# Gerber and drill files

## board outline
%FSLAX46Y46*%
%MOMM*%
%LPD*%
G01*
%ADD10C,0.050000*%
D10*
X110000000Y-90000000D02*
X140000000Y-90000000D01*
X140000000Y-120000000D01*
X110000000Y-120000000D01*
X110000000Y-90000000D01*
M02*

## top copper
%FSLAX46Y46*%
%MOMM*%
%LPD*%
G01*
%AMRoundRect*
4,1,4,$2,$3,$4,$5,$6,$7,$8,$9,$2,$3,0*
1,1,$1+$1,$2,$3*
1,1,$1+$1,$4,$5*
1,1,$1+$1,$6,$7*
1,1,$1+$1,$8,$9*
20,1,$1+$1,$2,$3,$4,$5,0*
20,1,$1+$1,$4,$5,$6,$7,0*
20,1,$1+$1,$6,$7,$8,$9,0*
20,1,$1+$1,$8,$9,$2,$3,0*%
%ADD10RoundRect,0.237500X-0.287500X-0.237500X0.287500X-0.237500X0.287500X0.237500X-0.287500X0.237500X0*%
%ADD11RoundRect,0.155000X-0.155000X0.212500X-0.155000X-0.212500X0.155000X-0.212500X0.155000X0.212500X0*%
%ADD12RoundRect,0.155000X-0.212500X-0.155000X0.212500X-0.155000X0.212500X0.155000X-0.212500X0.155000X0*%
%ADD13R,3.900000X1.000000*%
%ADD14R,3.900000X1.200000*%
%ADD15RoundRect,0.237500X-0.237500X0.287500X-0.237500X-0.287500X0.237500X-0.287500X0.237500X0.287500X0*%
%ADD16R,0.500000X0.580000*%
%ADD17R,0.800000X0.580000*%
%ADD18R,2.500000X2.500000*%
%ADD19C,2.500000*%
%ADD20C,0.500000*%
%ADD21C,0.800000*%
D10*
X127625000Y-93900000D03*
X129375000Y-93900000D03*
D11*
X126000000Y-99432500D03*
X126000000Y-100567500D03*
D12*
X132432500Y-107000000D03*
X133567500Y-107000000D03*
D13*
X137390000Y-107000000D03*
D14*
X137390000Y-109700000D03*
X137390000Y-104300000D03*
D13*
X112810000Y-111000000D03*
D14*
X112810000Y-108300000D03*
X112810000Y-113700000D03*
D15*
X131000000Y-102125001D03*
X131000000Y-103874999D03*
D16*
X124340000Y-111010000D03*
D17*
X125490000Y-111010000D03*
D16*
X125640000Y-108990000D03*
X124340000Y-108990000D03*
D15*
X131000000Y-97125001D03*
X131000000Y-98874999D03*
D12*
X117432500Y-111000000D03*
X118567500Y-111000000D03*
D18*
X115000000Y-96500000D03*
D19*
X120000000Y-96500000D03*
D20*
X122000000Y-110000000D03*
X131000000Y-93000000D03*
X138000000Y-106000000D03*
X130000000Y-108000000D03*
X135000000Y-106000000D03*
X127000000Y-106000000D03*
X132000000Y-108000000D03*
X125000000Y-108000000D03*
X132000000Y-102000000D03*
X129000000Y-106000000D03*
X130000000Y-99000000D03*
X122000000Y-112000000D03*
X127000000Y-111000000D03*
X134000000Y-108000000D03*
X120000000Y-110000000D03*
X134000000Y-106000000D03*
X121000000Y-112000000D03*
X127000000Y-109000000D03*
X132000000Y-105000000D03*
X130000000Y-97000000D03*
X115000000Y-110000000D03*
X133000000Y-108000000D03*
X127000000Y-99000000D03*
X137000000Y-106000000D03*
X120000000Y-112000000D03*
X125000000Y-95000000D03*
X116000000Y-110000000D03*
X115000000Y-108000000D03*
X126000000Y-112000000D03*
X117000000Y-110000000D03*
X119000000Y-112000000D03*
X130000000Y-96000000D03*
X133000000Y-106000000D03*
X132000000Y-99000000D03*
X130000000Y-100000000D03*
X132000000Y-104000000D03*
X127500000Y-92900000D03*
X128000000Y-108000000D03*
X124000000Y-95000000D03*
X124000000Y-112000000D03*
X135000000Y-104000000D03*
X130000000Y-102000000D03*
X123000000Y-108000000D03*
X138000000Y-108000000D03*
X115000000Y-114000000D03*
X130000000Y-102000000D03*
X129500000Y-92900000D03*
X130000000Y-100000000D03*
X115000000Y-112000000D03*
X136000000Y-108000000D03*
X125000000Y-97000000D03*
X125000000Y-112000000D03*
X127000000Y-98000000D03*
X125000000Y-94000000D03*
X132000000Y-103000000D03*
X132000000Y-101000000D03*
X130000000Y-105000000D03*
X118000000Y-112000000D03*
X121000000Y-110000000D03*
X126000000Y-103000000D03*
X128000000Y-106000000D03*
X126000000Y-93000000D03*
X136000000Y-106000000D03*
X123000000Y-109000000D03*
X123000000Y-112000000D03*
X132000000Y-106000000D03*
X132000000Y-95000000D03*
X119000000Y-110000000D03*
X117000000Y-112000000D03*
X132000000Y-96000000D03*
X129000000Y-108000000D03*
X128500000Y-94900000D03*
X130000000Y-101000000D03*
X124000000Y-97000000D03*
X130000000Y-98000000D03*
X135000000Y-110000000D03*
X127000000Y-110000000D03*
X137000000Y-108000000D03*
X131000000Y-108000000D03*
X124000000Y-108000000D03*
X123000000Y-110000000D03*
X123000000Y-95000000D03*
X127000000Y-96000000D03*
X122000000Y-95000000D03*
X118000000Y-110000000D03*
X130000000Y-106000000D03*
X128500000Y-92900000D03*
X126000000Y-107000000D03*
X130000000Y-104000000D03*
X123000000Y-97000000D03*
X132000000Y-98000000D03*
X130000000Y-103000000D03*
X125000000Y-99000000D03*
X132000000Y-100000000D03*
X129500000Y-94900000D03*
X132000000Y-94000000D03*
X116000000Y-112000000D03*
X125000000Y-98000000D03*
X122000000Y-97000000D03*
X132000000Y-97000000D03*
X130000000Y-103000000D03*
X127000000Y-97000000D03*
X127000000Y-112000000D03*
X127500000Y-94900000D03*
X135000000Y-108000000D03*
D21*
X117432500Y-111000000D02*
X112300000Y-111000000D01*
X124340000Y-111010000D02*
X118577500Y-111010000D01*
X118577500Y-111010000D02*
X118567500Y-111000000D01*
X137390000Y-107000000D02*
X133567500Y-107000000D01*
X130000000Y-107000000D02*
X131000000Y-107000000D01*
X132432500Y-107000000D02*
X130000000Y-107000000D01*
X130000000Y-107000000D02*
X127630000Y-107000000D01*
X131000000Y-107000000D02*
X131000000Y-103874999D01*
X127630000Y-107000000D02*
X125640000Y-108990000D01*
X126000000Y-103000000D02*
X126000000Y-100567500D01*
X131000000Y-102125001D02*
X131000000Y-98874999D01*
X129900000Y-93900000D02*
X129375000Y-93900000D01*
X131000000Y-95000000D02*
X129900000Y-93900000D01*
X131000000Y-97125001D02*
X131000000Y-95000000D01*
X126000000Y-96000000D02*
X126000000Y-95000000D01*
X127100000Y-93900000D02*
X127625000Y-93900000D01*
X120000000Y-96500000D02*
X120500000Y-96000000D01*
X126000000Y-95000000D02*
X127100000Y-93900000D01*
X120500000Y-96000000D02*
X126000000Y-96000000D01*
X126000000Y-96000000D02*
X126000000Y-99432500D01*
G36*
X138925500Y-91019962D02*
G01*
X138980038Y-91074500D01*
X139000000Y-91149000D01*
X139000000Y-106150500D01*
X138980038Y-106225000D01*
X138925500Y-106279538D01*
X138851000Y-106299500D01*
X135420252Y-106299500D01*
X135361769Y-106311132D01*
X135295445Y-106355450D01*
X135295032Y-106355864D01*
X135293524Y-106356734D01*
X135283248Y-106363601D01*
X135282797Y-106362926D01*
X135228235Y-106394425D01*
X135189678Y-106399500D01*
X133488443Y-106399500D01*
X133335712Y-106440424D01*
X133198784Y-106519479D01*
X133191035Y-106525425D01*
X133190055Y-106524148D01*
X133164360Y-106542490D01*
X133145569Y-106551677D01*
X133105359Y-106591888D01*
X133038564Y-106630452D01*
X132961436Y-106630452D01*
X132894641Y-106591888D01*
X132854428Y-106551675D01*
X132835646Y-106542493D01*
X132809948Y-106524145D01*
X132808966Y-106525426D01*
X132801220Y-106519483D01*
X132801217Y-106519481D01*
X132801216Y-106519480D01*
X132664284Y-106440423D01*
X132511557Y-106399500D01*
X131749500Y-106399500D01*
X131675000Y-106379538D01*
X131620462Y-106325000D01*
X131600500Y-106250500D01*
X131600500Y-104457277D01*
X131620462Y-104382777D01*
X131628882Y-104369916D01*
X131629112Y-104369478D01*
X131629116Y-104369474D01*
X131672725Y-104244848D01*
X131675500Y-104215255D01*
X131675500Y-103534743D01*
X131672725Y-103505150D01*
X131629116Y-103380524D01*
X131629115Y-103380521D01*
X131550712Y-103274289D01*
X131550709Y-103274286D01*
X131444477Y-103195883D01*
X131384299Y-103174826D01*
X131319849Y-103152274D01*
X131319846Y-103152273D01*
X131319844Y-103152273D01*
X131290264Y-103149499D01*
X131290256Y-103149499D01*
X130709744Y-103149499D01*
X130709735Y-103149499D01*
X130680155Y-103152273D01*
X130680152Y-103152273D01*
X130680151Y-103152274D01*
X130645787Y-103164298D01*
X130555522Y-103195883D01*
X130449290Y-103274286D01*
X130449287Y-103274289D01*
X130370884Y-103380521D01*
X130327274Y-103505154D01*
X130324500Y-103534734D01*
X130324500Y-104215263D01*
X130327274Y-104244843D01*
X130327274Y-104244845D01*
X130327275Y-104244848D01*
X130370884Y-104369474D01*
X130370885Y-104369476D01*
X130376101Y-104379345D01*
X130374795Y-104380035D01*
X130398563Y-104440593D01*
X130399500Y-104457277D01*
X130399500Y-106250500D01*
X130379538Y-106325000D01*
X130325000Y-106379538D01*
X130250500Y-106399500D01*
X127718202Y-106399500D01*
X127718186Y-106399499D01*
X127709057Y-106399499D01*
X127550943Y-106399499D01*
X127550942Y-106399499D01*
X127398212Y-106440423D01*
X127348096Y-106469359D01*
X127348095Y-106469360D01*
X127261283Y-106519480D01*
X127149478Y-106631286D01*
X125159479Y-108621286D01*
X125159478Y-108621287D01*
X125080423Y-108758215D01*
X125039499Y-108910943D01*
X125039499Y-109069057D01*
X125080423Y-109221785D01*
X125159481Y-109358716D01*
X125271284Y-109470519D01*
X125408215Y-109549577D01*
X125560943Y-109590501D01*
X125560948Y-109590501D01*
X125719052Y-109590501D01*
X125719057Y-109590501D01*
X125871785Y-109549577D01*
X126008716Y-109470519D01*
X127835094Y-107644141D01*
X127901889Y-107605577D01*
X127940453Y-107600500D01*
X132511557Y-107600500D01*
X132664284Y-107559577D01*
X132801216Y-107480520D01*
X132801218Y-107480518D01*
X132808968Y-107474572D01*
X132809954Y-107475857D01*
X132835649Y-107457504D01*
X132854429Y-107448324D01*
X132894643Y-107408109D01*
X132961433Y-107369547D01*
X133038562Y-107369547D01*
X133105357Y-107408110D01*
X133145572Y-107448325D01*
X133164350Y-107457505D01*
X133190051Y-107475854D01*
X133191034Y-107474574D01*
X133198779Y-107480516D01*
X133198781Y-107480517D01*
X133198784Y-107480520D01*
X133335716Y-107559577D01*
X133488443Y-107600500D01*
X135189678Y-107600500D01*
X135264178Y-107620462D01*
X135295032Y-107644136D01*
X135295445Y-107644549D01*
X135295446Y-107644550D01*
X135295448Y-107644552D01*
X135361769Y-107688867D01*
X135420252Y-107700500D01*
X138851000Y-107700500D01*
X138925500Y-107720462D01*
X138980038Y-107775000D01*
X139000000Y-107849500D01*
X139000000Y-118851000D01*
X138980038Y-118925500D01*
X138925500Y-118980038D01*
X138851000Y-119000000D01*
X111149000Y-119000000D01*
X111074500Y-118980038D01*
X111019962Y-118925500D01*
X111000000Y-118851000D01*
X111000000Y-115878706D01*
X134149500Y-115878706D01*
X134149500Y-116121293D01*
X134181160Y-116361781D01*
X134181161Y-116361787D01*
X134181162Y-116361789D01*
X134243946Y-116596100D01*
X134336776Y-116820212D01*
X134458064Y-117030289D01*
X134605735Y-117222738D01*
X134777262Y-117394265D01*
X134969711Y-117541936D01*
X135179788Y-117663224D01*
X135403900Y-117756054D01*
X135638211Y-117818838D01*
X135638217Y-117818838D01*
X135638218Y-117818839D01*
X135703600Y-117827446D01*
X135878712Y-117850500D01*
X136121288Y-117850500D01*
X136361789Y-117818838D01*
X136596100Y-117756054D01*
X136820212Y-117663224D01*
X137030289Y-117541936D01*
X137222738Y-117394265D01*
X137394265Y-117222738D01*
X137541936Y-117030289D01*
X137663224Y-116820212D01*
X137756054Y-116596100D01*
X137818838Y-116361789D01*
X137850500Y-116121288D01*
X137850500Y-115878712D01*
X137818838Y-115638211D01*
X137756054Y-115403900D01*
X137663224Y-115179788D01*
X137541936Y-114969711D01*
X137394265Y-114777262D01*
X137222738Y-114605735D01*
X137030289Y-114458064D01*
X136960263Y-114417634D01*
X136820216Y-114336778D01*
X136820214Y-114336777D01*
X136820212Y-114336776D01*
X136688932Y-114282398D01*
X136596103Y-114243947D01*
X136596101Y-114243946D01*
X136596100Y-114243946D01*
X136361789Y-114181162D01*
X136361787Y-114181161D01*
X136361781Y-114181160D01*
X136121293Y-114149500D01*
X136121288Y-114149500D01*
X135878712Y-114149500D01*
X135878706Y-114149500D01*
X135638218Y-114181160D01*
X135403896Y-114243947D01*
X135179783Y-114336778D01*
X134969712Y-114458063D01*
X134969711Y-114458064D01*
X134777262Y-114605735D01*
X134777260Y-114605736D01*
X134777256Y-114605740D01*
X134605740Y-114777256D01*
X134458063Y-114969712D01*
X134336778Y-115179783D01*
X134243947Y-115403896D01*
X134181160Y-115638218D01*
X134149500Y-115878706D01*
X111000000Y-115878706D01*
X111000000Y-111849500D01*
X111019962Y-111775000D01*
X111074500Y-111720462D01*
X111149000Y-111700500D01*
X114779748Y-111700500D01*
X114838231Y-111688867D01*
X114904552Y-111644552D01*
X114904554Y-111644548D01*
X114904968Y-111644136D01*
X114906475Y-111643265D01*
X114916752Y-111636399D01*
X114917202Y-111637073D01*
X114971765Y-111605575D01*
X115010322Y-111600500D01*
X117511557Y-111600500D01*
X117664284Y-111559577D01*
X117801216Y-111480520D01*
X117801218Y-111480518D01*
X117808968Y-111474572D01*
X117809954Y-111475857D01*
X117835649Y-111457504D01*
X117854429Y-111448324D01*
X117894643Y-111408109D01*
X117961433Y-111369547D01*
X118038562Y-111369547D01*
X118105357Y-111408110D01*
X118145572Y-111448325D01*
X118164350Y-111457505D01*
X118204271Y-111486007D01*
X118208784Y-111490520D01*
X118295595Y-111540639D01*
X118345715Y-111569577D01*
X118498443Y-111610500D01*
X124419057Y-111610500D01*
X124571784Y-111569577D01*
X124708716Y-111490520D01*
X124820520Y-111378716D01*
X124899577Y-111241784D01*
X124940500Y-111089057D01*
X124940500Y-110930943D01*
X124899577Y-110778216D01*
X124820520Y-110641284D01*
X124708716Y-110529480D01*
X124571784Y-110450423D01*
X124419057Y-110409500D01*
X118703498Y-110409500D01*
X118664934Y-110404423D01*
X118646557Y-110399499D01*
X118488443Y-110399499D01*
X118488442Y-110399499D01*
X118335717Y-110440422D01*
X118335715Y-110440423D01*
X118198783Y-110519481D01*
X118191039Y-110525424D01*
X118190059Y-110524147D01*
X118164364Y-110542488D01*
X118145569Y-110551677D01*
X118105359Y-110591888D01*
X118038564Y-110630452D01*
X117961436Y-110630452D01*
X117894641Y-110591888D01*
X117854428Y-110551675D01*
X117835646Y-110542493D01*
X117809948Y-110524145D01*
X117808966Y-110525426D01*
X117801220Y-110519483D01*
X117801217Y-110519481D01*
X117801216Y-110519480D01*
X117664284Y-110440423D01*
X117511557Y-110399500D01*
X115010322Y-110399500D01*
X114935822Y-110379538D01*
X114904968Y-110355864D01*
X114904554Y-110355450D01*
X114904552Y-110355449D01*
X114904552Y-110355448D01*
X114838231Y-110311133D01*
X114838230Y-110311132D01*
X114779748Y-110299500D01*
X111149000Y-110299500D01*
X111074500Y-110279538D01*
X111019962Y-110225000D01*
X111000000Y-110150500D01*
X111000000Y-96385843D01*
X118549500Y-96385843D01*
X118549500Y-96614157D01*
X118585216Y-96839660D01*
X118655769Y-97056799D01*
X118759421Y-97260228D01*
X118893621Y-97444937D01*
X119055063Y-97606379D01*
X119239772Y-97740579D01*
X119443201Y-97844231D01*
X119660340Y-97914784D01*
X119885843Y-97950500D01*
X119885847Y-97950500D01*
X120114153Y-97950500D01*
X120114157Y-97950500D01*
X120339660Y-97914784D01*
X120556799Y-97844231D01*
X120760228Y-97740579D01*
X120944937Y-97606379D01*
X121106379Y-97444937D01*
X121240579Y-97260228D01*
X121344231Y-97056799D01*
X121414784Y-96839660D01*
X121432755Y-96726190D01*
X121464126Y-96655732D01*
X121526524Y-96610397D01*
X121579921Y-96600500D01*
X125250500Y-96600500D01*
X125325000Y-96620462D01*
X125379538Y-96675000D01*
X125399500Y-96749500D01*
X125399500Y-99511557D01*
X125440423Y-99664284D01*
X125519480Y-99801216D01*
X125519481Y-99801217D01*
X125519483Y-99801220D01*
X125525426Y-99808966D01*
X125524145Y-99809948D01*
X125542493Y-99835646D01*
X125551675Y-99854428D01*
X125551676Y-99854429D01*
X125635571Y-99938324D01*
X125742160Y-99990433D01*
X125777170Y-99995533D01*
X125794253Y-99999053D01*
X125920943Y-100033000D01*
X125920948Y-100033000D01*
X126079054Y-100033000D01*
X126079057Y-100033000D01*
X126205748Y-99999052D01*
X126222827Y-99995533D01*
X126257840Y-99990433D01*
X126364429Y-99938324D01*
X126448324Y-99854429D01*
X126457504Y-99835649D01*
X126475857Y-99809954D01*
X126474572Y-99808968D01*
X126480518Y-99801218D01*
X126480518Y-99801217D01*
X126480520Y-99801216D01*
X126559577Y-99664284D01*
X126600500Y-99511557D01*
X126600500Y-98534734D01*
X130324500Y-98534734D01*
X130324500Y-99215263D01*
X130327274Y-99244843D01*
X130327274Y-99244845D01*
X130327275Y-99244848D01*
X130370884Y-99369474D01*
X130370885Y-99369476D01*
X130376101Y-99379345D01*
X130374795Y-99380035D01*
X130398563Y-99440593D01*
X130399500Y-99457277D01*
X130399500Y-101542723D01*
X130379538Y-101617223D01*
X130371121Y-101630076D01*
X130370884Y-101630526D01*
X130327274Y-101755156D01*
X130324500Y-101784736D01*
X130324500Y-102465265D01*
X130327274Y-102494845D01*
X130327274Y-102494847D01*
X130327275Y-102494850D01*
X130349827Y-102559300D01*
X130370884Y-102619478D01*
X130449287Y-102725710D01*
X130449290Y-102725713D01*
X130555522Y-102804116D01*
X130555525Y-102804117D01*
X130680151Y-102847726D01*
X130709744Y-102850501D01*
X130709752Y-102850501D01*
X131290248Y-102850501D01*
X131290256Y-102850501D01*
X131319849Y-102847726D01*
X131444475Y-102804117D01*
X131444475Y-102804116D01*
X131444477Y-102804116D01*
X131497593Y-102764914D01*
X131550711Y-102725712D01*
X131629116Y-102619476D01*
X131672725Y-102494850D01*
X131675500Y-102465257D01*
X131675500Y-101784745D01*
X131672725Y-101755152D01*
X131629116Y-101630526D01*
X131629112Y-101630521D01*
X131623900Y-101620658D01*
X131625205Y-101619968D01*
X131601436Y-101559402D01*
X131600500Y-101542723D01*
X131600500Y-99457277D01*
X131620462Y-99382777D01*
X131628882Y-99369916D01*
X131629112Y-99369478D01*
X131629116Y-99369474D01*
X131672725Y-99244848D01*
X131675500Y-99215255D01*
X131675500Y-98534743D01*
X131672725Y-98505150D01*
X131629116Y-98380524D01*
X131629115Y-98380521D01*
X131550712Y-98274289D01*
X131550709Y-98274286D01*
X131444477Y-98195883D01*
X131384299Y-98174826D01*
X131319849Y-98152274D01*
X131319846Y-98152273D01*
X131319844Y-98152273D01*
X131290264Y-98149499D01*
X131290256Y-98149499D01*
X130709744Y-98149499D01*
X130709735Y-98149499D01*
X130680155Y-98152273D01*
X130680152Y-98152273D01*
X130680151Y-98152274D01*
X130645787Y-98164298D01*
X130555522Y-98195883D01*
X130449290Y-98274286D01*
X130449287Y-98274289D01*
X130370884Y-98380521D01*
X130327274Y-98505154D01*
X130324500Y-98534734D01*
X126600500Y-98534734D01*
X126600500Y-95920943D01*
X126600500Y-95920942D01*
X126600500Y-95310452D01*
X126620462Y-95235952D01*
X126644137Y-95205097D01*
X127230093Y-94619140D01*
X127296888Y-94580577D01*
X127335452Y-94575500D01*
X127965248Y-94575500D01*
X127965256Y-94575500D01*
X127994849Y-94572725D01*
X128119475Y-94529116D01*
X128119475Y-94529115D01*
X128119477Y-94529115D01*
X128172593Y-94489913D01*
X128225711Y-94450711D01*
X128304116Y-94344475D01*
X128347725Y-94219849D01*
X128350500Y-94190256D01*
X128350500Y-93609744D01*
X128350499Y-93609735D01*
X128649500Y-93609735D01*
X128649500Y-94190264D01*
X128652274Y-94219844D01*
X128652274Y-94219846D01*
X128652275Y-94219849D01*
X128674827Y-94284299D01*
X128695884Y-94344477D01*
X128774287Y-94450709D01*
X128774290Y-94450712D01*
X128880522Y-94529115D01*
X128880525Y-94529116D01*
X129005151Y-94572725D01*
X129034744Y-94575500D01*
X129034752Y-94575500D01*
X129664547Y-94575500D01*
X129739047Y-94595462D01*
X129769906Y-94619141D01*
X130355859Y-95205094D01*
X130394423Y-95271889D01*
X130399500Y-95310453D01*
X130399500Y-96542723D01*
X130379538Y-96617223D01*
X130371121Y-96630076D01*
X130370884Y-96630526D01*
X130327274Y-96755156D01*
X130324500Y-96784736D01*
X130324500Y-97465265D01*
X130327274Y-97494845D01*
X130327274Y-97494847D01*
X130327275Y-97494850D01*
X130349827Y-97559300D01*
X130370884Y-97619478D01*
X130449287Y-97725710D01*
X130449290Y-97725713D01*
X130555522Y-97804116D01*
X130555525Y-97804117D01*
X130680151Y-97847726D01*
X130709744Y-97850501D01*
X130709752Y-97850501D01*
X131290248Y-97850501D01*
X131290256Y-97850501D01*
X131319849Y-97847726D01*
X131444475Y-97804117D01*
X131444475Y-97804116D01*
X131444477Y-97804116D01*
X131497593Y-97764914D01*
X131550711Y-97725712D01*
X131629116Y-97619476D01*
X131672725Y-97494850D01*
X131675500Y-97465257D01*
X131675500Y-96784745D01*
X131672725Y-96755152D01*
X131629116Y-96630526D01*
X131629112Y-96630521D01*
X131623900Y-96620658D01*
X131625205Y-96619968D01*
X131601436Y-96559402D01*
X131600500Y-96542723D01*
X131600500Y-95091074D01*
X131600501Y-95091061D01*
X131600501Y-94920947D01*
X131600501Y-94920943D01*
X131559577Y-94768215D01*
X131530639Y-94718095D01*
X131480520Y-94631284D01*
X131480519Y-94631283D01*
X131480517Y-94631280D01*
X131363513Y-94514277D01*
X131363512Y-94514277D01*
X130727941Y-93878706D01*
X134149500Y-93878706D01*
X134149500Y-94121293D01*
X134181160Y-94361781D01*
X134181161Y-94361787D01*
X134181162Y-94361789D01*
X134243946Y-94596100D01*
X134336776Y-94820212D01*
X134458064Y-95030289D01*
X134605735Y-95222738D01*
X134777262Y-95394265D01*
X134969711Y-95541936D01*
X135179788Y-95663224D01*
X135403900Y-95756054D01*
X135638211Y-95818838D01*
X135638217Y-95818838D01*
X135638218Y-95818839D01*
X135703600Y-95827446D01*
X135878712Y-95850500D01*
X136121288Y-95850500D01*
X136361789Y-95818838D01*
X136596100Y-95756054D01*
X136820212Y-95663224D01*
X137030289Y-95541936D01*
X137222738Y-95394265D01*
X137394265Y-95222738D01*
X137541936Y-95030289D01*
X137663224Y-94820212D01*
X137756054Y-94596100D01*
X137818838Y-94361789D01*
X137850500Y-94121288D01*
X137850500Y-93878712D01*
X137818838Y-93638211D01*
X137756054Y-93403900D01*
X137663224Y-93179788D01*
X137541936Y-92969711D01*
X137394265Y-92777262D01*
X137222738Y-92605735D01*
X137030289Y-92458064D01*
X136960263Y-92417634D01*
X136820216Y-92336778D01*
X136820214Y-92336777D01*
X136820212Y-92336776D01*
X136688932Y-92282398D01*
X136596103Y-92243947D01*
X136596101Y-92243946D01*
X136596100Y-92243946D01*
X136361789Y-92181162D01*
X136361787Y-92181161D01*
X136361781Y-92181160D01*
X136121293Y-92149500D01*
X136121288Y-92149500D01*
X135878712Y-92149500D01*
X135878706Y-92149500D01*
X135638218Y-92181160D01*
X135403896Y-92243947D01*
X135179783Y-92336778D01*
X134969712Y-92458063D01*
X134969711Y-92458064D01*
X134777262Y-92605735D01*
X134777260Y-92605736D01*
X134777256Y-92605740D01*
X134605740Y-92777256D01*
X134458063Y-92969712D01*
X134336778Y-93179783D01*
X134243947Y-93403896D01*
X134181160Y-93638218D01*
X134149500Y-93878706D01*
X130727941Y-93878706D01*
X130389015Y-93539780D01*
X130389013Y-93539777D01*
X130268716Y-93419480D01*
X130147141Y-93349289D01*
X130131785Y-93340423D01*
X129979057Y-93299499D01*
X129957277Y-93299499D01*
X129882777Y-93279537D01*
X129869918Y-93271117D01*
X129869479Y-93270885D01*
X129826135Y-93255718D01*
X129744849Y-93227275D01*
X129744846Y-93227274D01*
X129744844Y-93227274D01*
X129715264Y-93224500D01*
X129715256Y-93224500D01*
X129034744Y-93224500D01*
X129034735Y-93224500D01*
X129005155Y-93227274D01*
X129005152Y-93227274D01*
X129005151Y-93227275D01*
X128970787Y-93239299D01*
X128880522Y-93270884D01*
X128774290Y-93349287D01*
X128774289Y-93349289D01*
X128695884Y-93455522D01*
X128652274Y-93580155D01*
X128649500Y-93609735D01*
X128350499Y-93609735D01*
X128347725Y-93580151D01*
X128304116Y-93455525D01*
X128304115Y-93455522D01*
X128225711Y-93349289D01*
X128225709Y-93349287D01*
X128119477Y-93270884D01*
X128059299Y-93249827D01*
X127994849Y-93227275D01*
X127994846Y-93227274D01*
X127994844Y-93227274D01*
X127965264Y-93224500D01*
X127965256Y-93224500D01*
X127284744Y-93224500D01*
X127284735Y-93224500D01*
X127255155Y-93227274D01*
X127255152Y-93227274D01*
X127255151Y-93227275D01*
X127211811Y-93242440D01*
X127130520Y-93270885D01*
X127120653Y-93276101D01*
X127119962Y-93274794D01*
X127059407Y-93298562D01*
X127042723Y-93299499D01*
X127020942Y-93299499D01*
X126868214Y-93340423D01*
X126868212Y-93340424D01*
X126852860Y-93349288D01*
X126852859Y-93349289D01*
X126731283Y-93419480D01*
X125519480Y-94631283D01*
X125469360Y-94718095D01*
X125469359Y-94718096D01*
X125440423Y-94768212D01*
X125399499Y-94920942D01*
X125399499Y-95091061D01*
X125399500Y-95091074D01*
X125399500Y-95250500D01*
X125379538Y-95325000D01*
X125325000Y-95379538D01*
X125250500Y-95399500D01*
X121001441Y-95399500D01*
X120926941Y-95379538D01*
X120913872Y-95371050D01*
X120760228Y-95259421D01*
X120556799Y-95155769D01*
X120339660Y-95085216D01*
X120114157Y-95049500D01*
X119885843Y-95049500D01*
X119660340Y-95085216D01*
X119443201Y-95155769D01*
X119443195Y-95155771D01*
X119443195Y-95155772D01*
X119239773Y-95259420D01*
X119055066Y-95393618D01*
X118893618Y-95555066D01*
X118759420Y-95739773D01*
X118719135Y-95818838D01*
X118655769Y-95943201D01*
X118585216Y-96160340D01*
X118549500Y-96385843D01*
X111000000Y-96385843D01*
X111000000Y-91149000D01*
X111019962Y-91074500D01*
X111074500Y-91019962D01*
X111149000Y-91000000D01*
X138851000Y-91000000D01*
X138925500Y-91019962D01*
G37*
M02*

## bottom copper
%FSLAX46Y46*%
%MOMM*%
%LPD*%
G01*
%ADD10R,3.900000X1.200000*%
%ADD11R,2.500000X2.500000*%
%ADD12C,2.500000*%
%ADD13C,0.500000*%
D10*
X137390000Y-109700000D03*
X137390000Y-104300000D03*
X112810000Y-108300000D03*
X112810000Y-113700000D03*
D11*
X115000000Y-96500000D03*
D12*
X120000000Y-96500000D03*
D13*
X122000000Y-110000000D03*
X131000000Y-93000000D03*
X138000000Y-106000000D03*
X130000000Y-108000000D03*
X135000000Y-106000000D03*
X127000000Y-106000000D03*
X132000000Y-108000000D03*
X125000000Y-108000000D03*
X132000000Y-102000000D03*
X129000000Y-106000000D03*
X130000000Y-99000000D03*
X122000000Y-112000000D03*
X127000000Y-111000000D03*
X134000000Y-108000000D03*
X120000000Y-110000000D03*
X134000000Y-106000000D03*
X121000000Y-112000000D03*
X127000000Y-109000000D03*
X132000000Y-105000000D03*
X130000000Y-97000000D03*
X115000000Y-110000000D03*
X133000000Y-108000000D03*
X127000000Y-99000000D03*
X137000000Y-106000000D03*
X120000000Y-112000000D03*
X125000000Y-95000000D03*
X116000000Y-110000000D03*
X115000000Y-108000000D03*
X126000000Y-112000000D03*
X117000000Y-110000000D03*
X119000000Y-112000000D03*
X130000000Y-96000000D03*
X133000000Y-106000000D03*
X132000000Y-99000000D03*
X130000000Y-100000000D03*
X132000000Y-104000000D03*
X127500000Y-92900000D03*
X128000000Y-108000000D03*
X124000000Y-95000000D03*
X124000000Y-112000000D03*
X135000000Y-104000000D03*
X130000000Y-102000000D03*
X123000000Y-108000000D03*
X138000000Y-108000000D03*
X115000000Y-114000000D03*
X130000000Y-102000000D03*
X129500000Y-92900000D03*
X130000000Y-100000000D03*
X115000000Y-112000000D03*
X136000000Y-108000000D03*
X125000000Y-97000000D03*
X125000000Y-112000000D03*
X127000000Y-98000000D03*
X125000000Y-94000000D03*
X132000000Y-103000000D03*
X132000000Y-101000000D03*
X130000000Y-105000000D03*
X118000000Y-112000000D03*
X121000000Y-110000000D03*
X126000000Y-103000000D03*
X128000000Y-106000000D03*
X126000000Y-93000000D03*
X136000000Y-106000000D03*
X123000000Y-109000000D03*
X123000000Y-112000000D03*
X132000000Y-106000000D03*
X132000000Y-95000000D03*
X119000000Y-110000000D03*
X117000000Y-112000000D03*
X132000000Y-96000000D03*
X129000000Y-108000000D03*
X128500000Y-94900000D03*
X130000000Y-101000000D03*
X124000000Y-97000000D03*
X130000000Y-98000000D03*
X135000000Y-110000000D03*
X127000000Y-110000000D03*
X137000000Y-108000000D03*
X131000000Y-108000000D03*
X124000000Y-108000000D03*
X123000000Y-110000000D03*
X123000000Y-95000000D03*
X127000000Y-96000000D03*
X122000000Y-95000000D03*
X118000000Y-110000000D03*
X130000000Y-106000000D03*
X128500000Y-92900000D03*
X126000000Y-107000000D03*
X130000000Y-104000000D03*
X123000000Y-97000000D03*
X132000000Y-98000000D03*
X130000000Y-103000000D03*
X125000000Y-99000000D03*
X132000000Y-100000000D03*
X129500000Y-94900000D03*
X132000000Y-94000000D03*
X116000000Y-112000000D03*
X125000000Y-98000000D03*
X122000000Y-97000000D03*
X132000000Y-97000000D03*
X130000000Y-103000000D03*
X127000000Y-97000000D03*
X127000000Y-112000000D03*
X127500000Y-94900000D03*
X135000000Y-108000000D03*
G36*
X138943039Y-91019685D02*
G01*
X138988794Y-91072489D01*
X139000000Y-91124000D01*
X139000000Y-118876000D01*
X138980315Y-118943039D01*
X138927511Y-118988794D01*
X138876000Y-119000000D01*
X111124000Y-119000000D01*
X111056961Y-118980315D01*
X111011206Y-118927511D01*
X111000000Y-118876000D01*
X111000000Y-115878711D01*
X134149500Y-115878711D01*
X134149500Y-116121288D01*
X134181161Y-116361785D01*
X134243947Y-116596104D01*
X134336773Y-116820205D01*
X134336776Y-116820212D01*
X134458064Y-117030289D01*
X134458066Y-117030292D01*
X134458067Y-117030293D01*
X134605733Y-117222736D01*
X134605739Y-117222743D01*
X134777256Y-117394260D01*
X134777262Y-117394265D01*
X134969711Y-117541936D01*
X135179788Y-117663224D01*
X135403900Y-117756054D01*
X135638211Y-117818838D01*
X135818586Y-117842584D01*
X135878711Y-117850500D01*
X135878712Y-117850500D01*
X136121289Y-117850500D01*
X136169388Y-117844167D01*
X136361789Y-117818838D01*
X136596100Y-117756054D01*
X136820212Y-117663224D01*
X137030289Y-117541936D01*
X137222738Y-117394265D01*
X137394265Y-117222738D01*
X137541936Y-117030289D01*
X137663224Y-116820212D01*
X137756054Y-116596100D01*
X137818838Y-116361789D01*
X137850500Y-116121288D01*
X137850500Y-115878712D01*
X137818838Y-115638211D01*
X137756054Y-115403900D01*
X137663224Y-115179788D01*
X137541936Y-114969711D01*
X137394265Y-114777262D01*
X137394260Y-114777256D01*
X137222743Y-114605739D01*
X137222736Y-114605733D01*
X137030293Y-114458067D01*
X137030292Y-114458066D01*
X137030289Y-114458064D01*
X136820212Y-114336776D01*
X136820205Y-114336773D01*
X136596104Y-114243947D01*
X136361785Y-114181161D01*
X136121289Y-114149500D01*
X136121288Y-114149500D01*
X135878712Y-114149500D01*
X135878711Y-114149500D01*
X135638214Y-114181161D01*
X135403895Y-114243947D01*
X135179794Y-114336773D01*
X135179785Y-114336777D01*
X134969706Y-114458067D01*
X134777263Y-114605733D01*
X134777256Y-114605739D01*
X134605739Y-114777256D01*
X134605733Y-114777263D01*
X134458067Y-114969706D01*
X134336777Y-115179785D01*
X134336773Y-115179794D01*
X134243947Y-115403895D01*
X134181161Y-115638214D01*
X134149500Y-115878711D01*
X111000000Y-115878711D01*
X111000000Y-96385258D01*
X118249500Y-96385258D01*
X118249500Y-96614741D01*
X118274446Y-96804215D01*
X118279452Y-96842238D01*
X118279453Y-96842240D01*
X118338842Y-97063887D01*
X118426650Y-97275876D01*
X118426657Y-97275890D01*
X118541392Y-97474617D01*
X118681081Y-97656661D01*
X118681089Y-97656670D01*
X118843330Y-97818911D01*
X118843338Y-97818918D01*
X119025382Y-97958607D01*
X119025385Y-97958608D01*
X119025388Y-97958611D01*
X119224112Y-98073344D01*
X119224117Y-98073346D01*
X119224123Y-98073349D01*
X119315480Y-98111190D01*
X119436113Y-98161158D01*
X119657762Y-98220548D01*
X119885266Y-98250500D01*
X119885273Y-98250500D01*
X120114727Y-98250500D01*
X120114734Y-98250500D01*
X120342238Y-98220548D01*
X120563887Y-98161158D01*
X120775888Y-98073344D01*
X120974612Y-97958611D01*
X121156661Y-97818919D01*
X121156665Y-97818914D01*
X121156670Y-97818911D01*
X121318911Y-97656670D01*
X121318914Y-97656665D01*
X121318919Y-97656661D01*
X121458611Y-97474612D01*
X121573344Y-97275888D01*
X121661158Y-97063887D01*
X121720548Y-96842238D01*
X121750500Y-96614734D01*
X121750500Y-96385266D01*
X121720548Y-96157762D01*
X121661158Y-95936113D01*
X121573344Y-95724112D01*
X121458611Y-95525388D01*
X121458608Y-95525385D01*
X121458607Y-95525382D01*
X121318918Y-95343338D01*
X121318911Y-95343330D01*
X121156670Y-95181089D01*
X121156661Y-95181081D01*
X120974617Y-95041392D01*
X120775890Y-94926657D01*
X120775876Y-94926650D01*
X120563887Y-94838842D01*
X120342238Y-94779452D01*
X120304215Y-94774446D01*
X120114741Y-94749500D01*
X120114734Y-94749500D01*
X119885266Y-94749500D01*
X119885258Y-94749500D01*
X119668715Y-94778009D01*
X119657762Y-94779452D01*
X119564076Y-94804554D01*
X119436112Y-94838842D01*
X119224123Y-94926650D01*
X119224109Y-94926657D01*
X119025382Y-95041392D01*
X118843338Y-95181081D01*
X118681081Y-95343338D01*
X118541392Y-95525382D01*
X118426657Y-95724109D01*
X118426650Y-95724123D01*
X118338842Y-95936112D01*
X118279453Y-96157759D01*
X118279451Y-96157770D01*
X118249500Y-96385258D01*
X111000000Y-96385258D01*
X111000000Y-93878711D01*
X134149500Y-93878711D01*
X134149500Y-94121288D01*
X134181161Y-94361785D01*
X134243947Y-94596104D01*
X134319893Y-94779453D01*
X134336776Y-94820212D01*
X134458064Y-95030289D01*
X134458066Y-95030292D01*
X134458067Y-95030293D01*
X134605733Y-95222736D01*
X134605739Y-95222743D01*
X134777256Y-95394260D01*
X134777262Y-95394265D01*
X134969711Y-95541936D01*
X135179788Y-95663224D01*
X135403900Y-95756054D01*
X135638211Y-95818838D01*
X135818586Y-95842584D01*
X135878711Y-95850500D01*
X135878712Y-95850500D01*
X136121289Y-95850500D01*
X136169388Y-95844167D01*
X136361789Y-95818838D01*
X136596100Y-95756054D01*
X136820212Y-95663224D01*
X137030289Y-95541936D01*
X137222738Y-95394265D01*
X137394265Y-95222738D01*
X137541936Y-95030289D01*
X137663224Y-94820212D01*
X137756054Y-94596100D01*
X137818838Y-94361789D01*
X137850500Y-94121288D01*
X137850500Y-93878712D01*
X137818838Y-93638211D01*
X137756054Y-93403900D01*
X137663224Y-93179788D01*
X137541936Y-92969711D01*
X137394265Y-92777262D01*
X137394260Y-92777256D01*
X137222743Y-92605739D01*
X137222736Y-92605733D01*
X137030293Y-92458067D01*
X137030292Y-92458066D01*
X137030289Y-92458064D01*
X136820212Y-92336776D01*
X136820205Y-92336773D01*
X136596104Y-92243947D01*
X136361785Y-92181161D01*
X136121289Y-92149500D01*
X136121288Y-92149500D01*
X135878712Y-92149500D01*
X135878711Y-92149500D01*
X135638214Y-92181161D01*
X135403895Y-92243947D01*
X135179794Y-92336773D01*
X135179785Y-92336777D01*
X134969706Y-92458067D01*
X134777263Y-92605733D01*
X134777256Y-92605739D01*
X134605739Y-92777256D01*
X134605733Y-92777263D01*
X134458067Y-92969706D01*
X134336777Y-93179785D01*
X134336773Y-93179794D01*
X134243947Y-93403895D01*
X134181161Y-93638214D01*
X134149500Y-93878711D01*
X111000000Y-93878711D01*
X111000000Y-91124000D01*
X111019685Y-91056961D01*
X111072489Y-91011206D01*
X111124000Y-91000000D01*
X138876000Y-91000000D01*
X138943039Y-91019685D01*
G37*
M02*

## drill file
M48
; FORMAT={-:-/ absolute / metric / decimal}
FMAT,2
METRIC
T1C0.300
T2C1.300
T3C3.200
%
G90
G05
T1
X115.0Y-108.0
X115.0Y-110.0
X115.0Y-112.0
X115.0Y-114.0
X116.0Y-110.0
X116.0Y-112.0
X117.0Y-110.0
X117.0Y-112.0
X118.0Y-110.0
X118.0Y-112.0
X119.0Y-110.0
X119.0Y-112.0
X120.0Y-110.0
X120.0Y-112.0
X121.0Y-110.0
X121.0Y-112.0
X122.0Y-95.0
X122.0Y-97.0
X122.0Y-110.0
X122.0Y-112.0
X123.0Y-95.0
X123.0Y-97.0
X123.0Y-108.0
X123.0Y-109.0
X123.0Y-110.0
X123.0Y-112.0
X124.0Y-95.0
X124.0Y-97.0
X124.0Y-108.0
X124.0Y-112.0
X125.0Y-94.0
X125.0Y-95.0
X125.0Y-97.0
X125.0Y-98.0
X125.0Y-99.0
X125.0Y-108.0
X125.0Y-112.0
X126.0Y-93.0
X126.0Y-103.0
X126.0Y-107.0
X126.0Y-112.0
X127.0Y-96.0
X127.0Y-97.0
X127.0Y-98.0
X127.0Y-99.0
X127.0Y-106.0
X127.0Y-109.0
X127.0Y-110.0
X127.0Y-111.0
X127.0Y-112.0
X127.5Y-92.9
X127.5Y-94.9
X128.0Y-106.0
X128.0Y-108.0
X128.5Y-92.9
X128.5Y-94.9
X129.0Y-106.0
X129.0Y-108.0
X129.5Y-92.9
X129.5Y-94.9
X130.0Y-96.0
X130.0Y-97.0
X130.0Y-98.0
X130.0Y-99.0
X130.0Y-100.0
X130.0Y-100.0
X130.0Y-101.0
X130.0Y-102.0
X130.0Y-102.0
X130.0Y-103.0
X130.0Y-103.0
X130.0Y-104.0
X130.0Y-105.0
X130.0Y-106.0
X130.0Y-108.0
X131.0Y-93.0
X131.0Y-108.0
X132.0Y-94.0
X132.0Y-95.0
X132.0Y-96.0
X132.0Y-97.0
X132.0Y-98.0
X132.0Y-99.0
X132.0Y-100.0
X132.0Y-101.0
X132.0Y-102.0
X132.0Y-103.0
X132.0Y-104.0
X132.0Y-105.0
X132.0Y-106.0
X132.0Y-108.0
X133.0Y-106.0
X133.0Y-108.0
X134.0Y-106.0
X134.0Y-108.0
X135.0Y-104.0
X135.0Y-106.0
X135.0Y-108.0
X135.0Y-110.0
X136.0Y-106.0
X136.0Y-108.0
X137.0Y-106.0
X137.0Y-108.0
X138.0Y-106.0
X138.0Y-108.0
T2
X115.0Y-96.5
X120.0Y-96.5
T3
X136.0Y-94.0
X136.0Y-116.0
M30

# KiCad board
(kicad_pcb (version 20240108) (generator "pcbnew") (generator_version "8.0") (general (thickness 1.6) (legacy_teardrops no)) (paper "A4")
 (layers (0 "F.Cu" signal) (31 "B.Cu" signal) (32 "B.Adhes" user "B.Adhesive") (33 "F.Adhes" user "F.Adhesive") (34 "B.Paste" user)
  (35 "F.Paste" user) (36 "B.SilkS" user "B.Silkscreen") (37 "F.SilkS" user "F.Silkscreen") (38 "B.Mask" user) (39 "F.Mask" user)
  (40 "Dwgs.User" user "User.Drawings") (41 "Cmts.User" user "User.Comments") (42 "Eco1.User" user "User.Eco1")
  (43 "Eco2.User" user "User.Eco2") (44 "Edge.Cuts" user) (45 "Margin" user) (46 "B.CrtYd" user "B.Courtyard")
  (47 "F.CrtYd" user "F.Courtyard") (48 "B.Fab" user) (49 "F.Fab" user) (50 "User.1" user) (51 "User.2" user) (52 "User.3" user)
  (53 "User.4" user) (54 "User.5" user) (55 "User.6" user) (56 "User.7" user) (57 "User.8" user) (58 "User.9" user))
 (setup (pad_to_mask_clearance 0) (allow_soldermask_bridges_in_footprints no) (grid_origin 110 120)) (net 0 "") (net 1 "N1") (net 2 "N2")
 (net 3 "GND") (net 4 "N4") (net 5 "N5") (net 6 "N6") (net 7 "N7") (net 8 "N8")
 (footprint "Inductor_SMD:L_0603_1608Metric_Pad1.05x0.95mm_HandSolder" (layer "F.Cu") (at 128.5 93.9)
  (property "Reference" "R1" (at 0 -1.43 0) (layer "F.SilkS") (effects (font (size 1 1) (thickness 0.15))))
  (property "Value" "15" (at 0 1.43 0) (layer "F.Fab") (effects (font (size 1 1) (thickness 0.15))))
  (pad "1" smd roundrect (at -0.875 0) (size 1.05 0.95) (layers "F.Cu" "F.Paste" "F.Mask") (roundrect_rratio 0.25) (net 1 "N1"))
  (pad "2" smd roundrect (at 0.875 0) (size 1.05 0.95) (layers "F.Cu" "F.Paste" "F.Mask") (roundrect_rratio 0.25) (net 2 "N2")))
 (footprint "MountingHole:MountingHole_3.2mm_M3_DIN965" (layer "F.Cu") (at 136 94)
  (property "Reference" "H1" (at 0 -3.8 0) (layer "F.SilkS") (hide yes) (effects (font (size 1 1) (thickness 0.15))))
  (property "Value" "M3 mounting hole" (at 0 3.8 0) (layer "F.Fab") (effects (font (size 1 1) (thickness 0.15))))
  (pad "" np_thru_hole circle (at 0 0) (size 3.2 3.2) (drill 3.2) (layers "*.Cu" "*.Mask")))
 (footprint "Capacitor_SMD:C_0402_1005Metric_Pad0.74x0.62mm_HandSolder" (layer "F.Cu") (at 126 100 -90)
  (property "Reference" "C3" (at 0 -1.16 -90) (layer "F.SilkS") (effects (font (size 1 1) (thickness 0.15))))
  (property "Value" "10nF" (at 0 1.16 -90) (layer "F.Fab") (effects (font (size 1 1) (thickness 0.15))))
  (pad "1" smd roundrect (at -0.5675 0 270) (size 0.735 0.62) (layers "F.Cu" "F.Paste" "F.Mask") (roundrect_rratio 0.25) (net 1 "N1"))
  (pad "2" smd roundrect (at 0.5675 0 270) (size 0.735 0.62) (layers "F.Cu" "F.Paste" "F.Mask") (roundrect_rratio 0.25) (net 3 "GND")))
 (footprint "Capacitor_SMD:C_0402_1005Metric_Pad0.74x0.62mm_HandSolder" (layer "F.Cu") (at 133 107)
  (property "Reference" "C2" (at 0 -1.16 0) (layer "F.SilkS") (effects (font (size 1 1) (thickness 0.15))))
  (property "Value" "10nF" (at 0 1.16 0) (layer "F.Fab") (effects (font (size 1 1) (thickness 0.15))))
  (pad "1" smd roundrect (at -0.5675 0) (size 0.735 0.62) (layers "F.Cu" "F.Paste" "F.Mask") (roundrect_rratio 0.25) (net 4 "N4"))
  (pad "2" smd roundrect (at 0.5675 0) (size 0.735 0.62) (layers "F.Cu" "F.Paste" "F.Mask") (roundrect_rratio 0.25) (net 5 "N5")))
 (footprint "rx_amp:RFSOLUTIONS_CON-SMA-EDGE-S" (layer "F.Cu") (at 138.69 107 180)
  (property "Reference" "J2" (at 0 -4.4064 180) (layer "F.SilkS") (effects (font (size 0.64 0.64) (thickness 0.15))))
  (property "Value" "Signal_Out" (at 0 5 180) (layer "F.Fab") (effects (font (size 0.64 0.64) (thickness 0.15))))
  (pad "1" smd rect (at 1.3 0 180) (size 3.9 1) (layers "F.Cu" "F.Paste" "F.Mask") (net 5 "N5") (solder_mask_margin 0.102))
  (pad "2" smd rect (at 1.3 -2.7 180) (size 3.9 1.2) (layers "F.Cu" "F.Paste" "F.Mask") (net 3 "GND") (solder_mask_margin 0.102))
  (pad "2" smd rect (at 1.3 -2.7 180) (size 3.9 1.2) (layers "B.Cu" "B.Paste" "B.Mask") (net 3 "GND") (solder_mask_margin 0.102))
  (pad "2" smd rect (at 1.3 2.7 180) (size 3.9 1.2) (layers "F.Cu" "F.Paste" "F.Mask") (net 3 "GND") (solder_mask_margin 0.102))
  (pad "2" smd rect (at 1.3 2.7 180) (size 3.9 1.2) (layers "B.Cu" "B.Paste" "B.Mask") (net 3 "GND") (solder_mask_margin 0.102)))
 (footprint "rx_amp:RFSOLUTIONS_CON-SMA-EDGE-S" (layer "F.Cu") (at 111.51 111)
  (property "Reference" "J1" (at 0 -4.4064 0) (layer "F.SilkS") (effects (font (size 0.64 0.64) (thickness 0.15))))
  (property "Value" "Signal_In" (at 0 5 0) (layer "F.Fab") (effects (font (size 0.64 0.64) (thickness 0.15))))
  (pad "1" smd rect (at 1.3 0) (size 3.9 1) (layers "F.Cu" "F.Paste" "F.Mask") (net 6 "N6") (solder_mask_margin 0.102))
  (pad "2" smd rect (at 1.3 -2.7) (size 3.9 1.2) (layers "F.Cu" "F.Paste" "F.Mask") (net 3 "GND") (solder_mask_margin 0.102))
  (pad "2" smd rect (at 1.3 -2.7) (size 3.9 1.2) (layers "B.Cu" "B.Paste" "B.Mask") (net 3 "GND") (solder_mask_margin 0.102))
  (pad "2" smd rect (at 1.3 2.7) (size 3.9 1.2) (layers "F.Cu" "F.Paste" "F.Mask") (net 3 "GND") (solder_mask_margin 0.102))
  (pad "2" smd rect (at 1.3 2.7) (size 3.9 1.2) (layers "B.Cu" "B.Paste" "B.Mask") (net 3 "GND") (solder_mask_margin 0.102)))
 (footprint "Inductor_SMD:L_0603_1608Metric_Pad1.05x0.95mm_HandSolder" (layer "F.Cu") (at 131 103 -90)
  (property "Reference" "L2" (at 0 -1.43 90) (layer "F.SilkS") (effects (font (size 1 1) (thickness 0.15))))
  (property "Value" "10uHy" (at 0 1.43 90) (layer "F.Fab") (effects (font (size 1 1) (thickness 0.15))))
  (pad "1" smd roundrect (at -0.874999 0 270) (size 1.05 0.95) (layers "F.Cu" "F.Paste" "F.Mask") (roundrect_rratio 0.25) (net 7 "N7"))
  (pad "2" smd roundrect (at 0.874999 0 270) (size 1.05 0.95) (layers "F.Cu" "F.Paste" "F.Mask") (roundrect_rratio 0.25) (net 4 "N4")))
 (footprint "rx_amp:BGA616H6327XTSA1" (layer "F.Cu") (at 124.99 110)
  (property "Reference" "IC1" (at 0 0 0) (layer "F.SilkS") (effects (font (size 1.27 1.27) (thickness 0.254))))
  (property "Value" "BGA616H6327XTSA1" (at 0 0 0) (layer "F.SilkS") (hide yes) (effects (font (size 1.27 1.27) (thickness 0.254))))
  (pad "1" smd rect (at -0.65 1.01) (size 0.5 0.58) (layers "F.Cu" "F.Paste" "F.Mask") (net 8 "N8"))
  (pad "2" smd rect (at 0.5 1.01 90) (size 0.58 0.8) (layers "F.Cu" "F.Paste" "F.Mask") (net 3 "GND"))
  (pad "3" smd rect (at 0.65 -1.01) (size 0.5 0.58) (layers "F.Cu" "F.Paste" "F.Mask") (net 4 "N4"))
  (pad "4" smd rect (at -0.65 -1.01) (size 0.5 0.58) (layers "F.Cu" "F.Paste" "F.Mask") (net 3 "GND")))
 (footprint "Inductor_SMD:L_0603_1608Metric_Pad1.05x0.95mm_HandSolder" (layer "F.Cu") (at 131 98 -90)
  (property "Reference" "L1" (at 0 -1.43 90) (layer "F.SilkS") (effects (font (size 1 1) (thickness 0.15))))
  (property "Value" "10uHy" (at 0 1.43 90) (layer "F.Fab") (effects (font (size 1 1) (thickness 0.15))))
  (pad "1" smd roundrect (at -0.874999 0 270) (size 1.05 0.95) (layers "F.Cu" "F.Paste" "F.Mask") (roundrect_rratio 0.25) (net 2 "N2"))
  (pad "2" smd roundrect (at 0.874999 0 270) (size 1.05 0.95) (layers "F.Cu" "F.Paste" "F.Mask") (roundrect_rratio 0.25) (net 7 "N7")))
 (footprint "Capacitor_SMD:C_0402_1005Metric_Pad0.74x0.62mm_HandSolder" (layer "F.Cu") (at 118 111)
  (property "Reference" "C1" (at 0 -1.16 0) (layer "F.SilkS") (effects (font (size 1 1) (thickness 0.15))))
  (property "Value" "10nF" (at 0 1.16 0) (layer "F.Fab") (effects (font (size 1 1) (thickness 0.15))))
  (pad "1" smd roundrect (at -0.5675 0) (size 0.735 0.62) (layers "F.Cu" "F.Paste" "F.Mask") (roundrect_rratio 0.25) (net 6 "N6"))
  (pad "2" smd roundrect (at 0.5675 0) (size 0.735 0.62) (layers "F.Cu" "F.Paste" "F.Mask") (roundrect_rratio 0.25) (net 8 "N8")))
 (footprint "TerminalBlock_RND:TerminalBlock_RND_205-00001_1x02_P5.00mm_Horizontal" (layer "F.Cu") (at 115 96.5)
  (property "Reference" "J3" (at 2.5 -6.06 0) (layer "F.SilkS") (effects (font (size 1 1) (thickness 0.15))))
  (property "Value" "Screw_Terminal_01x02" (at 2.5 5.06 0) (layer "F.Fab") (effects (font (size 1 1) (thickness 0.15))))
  (pad "1" thru_hole rect (at 0 0) (size 2.5 2.5) (drill 1.3) (layers "*.Cu" "*.Mask") (remove_unused_layers no) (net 3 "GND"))
  (pad "2" thru_hole circle (at 5 0) (size 2.5 2.5) (drill 1.3) (layers "*.Cu" "*.Mask") (remove_unused_layers no) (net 1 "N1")))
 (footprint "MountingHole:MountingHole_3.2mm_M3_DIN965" (layer "F.Cu") (at 136 116)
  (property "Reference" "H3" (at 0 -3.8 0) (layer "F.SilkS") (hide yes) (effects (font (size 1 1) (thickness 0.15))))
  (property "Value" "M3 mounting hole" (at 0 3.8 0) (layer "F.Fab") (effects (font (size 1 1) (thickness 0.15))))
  (pad "" np_thru_hole circle (at 0 0) (size 3.2 3.2) (drill 3.2) (layers "*.Cu" "*.Mask")))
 (gr_rect (start 110 90) (end 140 120) (stroke (width 0.05) (type default)) (fill none) (layer "Edge.Cuts"))
 (segment (start 117.4325 111) (end 112.3 111) (width 0.8) (layer "F.Cu") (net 6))
 (segment (start 124.34 111.01) (end 118.5775 111.01) (width 0.8) (layer "F.Cu") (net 8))
 (segment (start 118.5775 111.01) (end 118.5675 111) (width 0.8) (layer "F.Cu") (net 8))
 (segment (start 137.39 107) (end 133.5675 107) (width 0.8) (layer "F.Cu") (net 5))
 (segment (start 130 107) (end 131 107) (width 0.8) (layer "F.Cu") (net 4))
 (segment (start 132.4325 107) (end 130 107) (width 0.8) (layer "F.Cu") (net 4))
 (segment (start 130 107) (end 127.63 107) (width 0.8) (layer "F.Cu") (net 4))
 (segment (start 131 107) (end 131 103.874999) (width 0.8) (layer "F.Cu") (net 4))
 (segment (start 127.63 107) (end 125.64 108.99) (width 0.8) (layer "F.Cu") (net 4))
 (segment (start 126 103) (end 126 100.5675) (width 0.8) (layer "F.Cu") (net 3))
 (via (at 122 110) (size 0.5) (drill 0.3) (layers "F.Cu" "B.Cu") (free yes) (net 3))
 (via (at 131 93) (size 0.5) (drill 0.3) (layers "F.Cu" "B.Cu") (free yes) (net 3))
 (via (at 138 106) (size 0.5) (drill 0.3) (layers "F.Cu" "B.Cu") (free yes) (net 3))
 (via (at 130 108) (size 0.5) (drill 0.3) (layers "F.Cu" "B.Cu") (free yes) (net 3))
 (via (at 135 106) (size 0.5) (drill 0.3) (layers "F.Cu" "B.Cu") (free yes) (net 3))
 (via (at 127 106) (size 0.5) (drill 0.3) (layers "F.Cu" "B.Cu") (free yes) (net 3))
 (via (at 132 108) (size 0.5) (drill 0.3) (layers "F.Cu" "B.Cu") (free yes) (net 3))
 (via (at 125 108) (size 0.5) (drill 0.3) (layers "F.Cu" "B.Cu") (free yes) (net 3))
 (via (at 132 102) (size 0.5) (drill 0.3) (layers "F.Cu" "B.Cu") (free yes) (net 3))
 (via (at 129 106) (size 0.5) (drill 0.3) (layers "F.Cu" "B.Cu") (free yes) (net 3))
 (via (at 130 99) (size 0.5) (drill 0.3) (layers "F.Cu" "B.Cu") (free yes) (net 3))
 (via (at 122 112) (size 0.5) (drill 0.3) (layers "F.Cu" "B.Cu") (free yes) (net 3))
 (via (at 127 111) (size 0.5) (drill 0.3) (layers "F.Cu" "B.Cu") (free yes) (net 3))
 (via (at 134 108) (size 0.5) (drill 0.3) (layers "F.Cu" "B.Cu") (free yes) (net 3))
 (via (at 120 110) (size 0.5) (drill 0.3) (layers "F.Cu" "B.Cu") (free yes) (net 3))
 (via (at 134 106) (size 0.5) (drill 0.3) (layers "F.Cu" "B.Cu") (free yes) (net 3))
 (via (at 121 112) (size 0.5) (drill 0.3) (layers "F.Cu" "B.Cu") (free yes) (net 3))
 (via (at 127 109) (size 0.5) (drill 0.3) (layers "F.Cu" "B.Cu") (free yes) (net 3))
 (via (at 132 105) (size 0.5) (drill 0.3) (layers "F.Cu" "B.Cu") (free yes) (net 3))
 (via (at 130 97) (size 0.5) (drill 0.3) (layers "F.Cu" "B.Cu") (free yes) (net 3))
 (via (at 115 110) (size 0.5) (drill 0.3) (layers "F.Cu" "B.Cu") (free yes) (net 3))
 (via (at 133 108) (size 0.5) (drill 0.3) (layers "F.Cu" "B.Cu") (free yes) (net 3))
 (via (at 127 99) (size 0.5) (drill 0.3) (layers "F.Cu" "B.Cu") (free yes) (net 3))
 (via (at 137 106) (size 0.5) (drill 0.3) (layers "F.Cu" "B.Cu") (free yes) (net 3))
 (via (at 120 112) (size 0.5) (drill 0.3) (layers "F.Cu" "B.Cu") (free yes) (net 3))
 (via (at 125 95) (size 0.5) (drill 0.3) (layers "F.Cu" "B.Cu") (free yes) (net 3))
 (via (at 116 110) (size 0.5) (drill 0.3) (layers "F.Cu" "B.Cu") (free yes) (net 3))
 (via (at 115 108) (size 0.5) (drill 0.3) (layers "F.Cu" "B.Cu") (free yes) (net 3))
 (via (at 126 112) (size 0.5) (drill 0.3) (layers "F.Cu" "B.Cu") (free yes) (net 3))
 (via (at 117 110) (size 0.5) (drill 0.3) (layers "F.Cu" "B.Cu") (free yes) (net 3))
 (via (at 119 112) (size 0.5) (drill 0.3) (layers "F.Cu" "B.Cu") (free yes) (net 3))
 (via (at 130 96) (size 0.5) (drill 0.3) (layers "F.Cu" "B.Cu") (free yes) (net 3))
 (via (at 133 106) (size 0.5) (drill 0.3) (layers "F.Cu" "B.Cu") (free yes) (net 3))
 (via (at 132 99) (size 0.5) (drill 0.3) (layers "F.Cu" "B.Cu") (free yes) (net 3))
 (via (at 130 100) (size 0.5) (drill 0.3) (layers "F.Cu" "B.Cu") (free yes) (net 3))
 (via (at 132 104) (size 0.5) (drill 0.3) (layers "F.Cu" "B.Cu") (free yes) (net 3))
 (via (at 127.5 92.9) (size 0.5) (drill 0.3) (layers "F.Cu" "B.Cu") (free yes) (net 3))
 (via (at 128 108) (size 0.5) (drill 0.3) (layers "F.Cu" "B.Cu") (free yes) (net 3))
 (via (at 124 95) (size 0.5) (drill 0.3) (layers "F.Cu" "B.Cu") (free yes) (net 3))
 (via (at 124 112) (size 0.5) (drill 0.3) (layers "F.Cu" "B.Cu") (free yes) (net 3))
 (via (at 135 104) (size 0.5) (drill 0.3) (layers "F.Cu" "B.Cu") (free yes) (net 3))
 (via (at 130 102) (size 0.5) (drill 0.3) (layers "F.Cu" "B.Cu") (free yes) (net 3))
 (via (at 123 108) (size 0.5) (drill 0.3) (layers "F.Cu" "B.Cu") (free yes) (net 3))
 (via (at 138 108) (size 0.5) (drill 0.3) (layers "F.Cu" "B.Cu") (free yes) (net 3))
 (via (at 115 114) (size 0.5) (drill 0.3) (layers "F.Cu" "B.Cu") (free yes) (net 3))
 (via (at 130 102) (size 0.5) (drill 0.3) (layers "F.Cu" "B.Cu") (free yes) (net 3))
 (via (at 129.5 92.9) (size 0.5) (drill 0.3) (layers "F.Cu" "B.Cu") (free yes) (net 3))
 (via (at 130 100) (size 0.5) (drill 0.3) (layers "F.Cu" "B.Cu") (free yes) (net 3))
 (via (at 115 112) (size 0.5) (drill 0.3) (layers "F.Cu" "B.Cu") (free yes) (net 3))
 (via (at 136 108) (size 0.5) (drill 0.3) (layers "F.Cu" "B.Cu") (free yes) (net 3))
 (via (at 125 97) (size 0.5) (drill 0.3) (layers "F.Cu" "B.Cu") (free yes) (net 3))
 (via (at 125 112) (size 0.5) (drill 0.3) (layers "F.Cu" "B.Cu") (free yes) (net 3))
 (via (at 127 98) (size 0.5) (drill 0.3) (layers "F.Cu" "B.Cu") (free yes) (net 3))
 (via (at 125 94) (size 0.5) (drill 0.3) (layers "F.Cu" "B.Cu") (free yes) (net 3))
 (via (at 132 103) (size 0.5) (drill 0.3) (layers "F.Cu" "B.Cu") (free yes) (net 3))
 (via (at 132 101) (size 0.5) (drill 0.3) (layers "F.Cu" "B.Cu") (free yes) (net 3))
 (via (at 130 105) (size 0.5) (drill 0.3) (layers "F.Cu" "B.Cu") (free yes) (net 3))
 (via (at 118 112) (size 0.5) (drill 0.3) (layers "F.Cu" "B.Cu") (free yes) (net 3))
 (via (at 121 110) (size 0.5) (drill 0.3) (layers "F.Cu" "B.Cu") (free yes) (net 3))
 (via (at 126 103) (size 0.5) (drill 0.3) (layers "F.Cu" "B.Cu") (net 3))
 (via (at 128 106) (size 0.5) (drill 0.3) (layers "F.Cu" "B.Cu") (free yes) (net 3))
 (via (at 126 93) (size 0.5) (drill 0.3) (layers "F.Cu" "B.Cu") (free yes) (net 3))
 (via (at 136 106) (size 0.5) (drill 0.3) (layers "F.Cu" "B.Cu") (free yes) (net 3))
 (via (at 123 109) (size 0.5) (drill 0.3) (layers "F.Cu" "B.Cu") (free yes) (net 3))
 (via (at 123 112) (size 0.5) (drill 0.3) (layers "F.Cu" "B.Cu") (free yes) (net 3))
 (via (at 132 106) (size 0.5) (drill 0.3) (layers "F.Cu" "B.Cu") (free yes) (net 3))
 (via (at 132 95) (size 0.5) (drill 0.3) (layers "F.Cu" "B.Cu") (free yes) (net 3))
 (via (at 119 110) (size 0.5) (drill 0.3) (layers "F.Cu" "B.Cu") (free yes) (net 3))
 (via (at 117 112) (size 0.5) (drill 0.3) (layers "F.Cu" "B.Cu") (free yes) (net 3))
 (via (at 132 96) (size 0.5) (drill 0.3) (layers "F.Cu" "B.Cu") (free yes) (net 3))
 (via (at 129 108) (size 0.5) (drill 0.3) (layers "F.Cu" "B.Cu") (free yes) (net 3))
 (via (at 128.5 94.9) (size 0.5) (drill 0.3) (layers "F.Cu" "B.Cu") (free yes) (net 3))
 (via (at 130 101) (size 0.5) (drill 0.3) (layers "F.Cu" "B.Cu") (free yes) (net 3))
 (via (at 124 97) (size 0.5) (drill 0.3) (layers "F.Cu" "B.Cu") (free yes) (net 3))
 (via (at 130 98) (size 0.5) (drill 0.3) (layers "F.Cu" "B.Cu") (free yes) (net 3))
 (via (at 135 110) (size 0.5) (drill 0.3) (layers "F.Cu" "B.Cu") (free yes) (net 3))
 (via (at 127 110) (size 0.5) (drill 0.3) (layers "F.Cu" "B.Cu") (free yes) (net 3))
 (via (at 137 108) (size 0.5) (drill 0.3) (layers "F.Cu" "B.Cu") (free yes) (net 3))
 (via (at 131 108) (size 0.5) (drill 0.3) (layers "F.Cu" "B.Cu") (free yes) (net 3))
 (via (at 124 108) (size 0.5) (drill 0.3) (layers "F.Cu" "B.Cu") (free yes) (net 3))
 (via (at 123 110) (size 0.5) (drill 0.3) (layers "F.Cu" "B.Cu") (free yes) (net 3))
 (via (at 123 95) (size 0.5) (drill 0.3) (layers "F.Cu" "B.Cu") (free yes) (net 3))
 (via (at 127 96) (size 0.5) (drill 0.3) (layers "F.Cu" "B.Cu") (free yes) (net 3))
 (via (at 122 95) (size 0.5) (drill 0.3) (layers "F.Cu" "B.Cu") (free yes) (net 3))
 (via (at 118 110) (size 0.5) (drill 0.3) (layers "F.Cu" "B.Cu") (free yes) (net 3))
 (via (at 130 106) (size 0.5) (drill 0.3) (layers "F.Cu" "B.Cu") (free yes) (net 3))
 (via (at 128.5 92.9) (size 0.5) (drill 0.3) (layers "F.Cu" "B.Cu") (free yes) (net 3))
 (via (at 126 107) (size 0.5) (drill 0.3) (layers "F.Cu" "B.Cu") (free yes) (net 3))
 (via (at 130 104) (size 0.5) (drill 0.3) (layers "F.Cu" "B.Cu") (free yes) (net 3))
 (via (at 123 97) (size 0.5) (drill 0.3) (layers "F.Cu" "B.Cu") (free yes) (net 3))
 (via (at 132 98) (size 0.5) (drill 0.3) (layers "F.Cu" "B.Cu") (free yes) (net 3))
 (via (at 130 103) (size 0.5) (drill 0.3) (layers "F.Cu" "B.Cu") (free yes) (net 3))
 (via (at 125 99) (size 0.5) (drill 0.3) (layers "F.Cu" "B.Cu") (free yes) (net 3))
 (via (at 132 100) (size 0.5) (drill 0.3) (layers "F.Cu" "B.Cu") (free yes) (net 3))
 (via (at 129.5 94.9) (size 0.5) (drill 0.3) (layers "F.Cu" "B.Cu") (free yes) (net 3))
 (via (at 132 94) (size 0.5) (drill 0.3) (layers "F.Cu" "B.Cu") (free yes) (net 3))
 (via (at 116 112) (size 0.5) (drill 0.3) (layers "F.Cu" "B.Cu") (free yes) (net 3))
 (via (at 125 98) (size 0.5) (drill 0.3) (layers "F.Cu" "B.Cu") (free yes) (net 3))
 (via (at 122 97) (size 0.5) (drill 0.3) (layers "F.Cu" "B.Cu") (free yes) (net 3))
 (via (at 132 97) (size 0.5) (drill 0.3) (layers "F.Cu" "B.Cu") (free yes) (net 3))
 (via (at 130 103) (size 0.5) (drill 0.3) (layers "F.Cu" "B.Cu") (free yes) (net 3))
 (via (at 127 97) (size 0.5) (drill 0.3) (layers "F.Cu" "B.Cu") (free yes) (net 3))
 (via (at 127 112) (size 0.5) (drill 0.3) (layers "F.Cu" "B.Cu") (free yes) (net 3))
 (via (at 127.5 94.9) (size 0.5) (drill 0.3) (layers "F.Cu" "B.Cu") (free yes) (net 3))
 (via (at 135 108) (size 0.5) (drill 0.3) (layers "F.Cu" "B.Cu") (free yes) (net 3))
 (segment (start 131 102.125001) (end 131 98.874999) (width 0.8) (layer "F.Cu") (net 7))
 (segment (start 129.9 93.9) (end 129.375 93.9) (width 0.8) (layer "F.Cu") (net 2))
 (segment (start 131 95) (end 129.9 93.9) (width 0.8) (layer "F.Cu") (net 2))
 (segment (start 131 97.125001) (end 131 95) (width 0.8) (layer "F.Cu") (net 2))
 (segment (start 126 96) (end 126 95) (width 0.8) (layer "F.Cu") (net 1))
 (segment (start 127.1 93.9) (end 127.625 93.9) (width 0.8) (layer "F.Cu") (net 1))
 (segment (start 120 96.5) (end 120.5 96) (width 0.8) (layer "F.Cu") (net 1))
 (segment (start 126 95) (end 127.1 93.9) (width 0.8) (layer "F.Cu") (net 1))
 (segment (start 120.5 96) (end 126 96) (width 0.8) (layer "F.Cu") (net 1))
 (segment (start 126 96) (end 126 99.4325) (width 0.8) (layer "F.Cu") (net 1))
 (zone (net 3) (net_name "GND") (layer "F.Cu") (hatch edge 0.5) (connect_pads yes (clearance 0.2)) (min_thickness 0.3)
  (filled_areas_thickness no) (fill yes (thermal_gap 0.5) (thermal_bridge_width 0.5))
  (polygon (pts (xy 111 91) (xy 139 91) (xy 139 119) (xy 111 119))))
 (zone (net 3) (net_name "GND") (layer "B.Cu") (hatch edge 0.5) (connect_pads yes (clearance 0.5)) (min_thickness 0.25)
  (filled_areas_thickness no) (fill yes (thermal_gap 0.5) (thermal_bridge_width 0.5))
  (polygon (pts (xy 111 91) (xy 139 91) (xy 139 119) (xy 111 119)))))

